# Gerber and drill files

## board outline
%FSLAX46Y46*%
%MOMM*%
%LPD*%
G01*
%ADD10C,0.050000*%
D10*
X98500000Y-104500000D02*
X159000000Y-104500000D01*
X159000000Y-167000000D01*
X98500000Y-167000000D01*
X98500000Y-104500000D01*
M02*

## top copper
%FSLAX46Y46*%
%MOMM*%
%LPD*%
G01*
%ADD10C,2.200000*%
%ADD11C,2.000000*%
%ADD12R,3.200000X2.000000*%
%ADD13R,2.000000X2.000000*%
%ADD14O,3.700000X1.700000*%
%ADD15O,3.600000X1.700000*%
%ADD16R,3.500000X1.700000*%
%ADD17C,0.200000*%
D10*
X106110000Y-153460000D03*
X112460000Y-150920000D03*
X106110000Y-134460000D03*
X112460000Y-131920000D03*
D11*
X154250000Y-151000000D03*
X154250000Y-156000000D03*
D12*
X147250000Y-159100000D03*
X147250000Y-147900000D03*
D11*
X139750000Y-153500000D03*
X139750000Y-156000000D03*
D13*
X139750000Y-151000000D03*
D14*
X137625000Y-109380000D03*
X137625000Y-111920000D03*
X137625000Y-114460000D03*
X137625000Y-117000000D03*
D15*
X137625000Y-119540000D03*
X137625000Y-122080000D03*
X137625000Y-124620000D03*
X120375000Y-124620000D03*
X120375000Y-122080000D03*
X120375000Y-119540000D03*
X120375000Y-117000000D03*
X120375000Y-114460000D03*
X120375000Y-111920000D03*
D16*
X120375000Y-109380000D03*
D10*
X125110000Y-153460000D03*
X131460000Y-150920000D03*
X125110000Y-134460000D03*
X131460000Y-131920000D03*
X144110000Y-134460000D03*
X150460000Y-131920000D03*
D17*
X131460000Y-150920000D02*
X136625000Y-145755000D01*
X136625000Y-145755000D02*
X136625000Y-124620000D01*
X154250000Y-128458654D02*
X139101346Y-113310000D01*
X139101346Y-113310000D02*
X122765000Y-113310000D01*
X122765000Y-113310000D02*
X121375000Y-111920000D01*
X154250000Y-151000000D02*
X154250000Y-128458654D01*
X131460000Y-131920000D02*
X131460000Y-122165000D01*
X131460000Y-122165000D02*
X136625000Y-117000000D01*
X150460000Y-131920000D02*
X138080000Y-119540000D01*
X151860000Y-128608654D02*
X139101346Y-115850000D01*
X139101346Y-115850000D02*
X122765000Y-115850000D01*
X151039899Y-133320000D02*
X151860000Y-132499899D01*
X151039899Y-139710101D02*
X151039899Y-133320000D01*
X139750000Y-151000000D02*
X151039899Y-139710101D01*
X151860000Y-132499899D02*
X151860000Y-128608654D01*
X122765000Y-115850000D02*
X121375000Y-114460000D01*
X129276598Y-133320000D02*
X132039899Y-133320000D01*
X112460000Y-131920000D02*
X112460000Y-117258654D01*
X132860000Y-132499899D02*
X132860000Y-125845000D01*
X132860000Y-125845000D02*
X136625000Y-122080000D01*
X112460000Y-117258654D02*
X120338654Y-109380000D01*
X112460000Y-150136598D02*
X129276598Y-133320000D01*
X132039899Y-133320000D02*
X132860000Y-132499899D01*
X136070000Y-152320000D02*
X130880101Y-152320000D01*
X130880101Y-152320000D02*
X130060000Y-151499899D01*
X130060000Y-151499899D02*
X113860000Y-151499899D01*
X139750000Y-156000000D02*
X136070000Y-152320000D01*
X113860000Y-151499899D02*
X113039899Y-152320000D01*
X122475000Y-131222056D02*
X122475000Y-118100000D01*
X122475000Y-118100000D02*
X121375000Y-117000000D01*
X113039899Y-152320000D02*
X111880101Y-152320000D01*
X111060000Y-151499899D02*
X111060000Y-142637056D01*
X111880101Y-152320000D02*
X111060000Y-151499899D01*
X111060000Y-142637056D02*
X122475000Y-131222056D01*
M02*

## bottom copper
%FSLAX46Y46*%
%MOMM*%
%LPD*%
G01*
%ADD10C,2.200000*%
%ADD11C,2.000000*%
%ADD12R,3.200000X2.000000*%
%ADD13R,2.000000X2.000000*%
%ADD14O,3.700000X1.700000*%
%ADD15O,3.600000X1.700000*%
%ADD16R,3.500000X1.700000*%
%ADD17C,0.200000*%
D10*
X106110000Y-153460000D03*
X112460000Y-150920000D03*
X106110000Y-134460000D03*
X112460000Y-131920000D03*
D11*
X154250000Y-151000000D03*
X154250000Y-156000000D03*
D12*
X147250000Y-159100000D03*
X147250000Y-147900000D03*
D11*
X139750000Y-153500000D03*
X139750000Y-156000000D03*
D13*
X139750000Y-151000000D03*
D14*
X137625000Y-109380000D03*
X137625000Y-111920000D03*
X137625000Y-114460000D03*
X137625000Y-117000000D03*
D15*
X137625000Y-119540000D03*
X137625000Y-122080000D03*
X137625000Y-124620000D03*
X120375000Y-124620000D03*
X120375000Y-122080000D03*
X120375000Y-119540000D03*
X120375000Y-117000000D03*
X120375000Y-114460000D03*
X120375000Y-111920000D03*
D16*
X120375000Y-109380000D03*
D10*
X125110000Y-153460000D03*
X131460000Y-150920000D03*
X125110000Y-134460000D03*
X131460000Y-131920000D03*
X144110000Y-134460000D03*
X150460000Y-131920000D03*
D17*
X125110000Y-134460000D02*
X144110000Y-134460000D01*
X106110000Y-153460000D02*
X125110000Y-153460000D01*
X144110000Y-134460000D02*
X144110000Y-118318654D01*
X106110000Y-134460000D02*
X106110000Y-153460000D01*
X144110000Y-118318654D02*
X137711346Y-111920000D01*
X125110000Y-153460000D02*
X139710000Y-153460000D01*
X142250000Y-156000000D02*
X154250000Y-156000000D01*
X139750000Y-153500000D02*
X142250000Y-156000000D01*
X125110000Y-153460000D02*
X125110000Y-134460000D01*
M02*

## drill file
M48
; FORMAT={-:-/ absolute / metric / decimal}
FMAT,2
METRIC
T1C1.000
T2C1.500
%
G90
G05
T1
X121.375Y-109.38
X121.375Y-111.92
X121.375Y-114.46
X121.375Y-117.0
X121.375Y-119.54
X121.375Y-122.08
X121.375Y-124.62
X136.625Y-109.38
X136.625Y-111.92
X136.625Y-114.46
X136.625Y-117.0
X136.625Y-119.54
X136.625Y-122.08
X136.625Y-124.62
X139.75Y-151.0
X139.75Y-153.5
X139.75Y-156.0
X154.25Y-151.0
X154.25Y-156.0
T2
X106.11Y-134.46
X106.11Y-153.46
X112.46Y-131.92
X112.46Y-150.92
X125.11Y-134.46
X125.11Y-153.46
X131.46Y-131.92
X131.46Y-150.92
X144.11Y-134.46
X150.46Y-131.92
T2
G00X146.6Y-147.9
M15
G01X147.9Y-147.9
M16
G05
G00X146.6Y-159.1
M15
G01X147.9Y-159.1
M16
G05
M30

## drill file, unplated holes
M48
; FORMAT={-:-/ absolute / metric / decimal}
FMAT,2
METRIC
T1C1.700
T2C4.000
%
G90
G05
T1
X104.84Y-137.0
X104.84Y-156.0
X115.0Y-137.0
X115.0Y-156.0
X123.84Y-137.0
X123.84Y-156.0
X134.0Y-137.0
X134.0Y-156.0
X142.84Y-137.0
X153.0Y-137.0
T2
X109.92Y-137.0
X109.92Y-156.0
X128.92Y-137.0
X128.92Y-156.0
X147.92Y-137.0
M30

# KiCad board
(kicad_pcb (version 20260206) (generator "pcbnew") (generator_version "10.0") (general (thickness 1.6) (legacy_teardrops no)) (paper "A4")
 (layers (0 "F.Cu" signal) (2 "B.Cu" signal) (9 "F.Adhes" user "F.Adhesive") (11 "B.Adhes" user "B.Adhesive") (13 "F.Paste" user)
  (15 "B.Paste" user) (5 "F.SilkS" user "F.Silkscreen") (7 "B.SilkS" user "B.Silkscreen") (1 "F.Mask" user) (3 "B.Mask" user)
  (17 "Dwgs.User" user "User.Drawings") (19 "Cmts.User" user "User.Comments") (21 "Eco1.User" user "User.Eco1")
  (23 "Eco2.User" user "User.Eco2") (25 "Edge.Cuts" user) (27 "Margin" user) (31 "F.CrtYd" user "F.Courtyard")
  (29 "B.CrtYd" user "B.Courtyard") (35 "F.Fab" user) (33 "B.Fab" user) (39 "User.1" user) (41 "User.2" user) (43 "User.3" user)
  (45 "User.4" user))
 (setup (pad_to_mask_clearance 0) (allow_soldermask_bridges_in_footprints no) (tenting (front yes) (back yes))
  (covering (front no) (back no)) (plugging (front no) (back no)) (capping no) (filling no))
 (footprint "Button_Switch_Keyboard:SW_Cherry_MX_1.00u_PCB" (layer "F.Cu") (at 112.46 150.92)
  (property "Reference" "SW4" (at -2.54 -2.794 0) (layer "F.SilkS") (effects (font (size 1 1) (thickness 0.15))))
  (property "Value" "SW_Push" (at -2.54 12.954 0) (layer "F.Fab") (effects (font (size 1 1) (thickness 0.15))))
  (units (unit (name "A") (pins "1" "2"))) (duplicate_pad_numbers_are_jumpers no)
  (pad "" np_thru_hole circle (at -7.62 5.08) (size 1.7 1.7) (drill 1.7) (layers "*.Cu" "*.Mask"))
  (pad "" np_thru_hole circle (at -2.54 5.08) (size 4 4) (drill 4) (layers "*.Cu" "*.Mask"))
  (pad "" np_thru_hole circle (at 2.54 5.08) (size 1.7 1.7) (drill 1.7) (layers "*.Cu" "*.Mask"))
  (pad "1" thru_hole circle (at 0 0) (size 2.2 2.2) (drill 1.5) (layers "*.Cu" "*.Mask") (remove_unused_layers no)
   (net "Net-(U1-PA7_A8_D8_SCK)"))
  (pad "2" thru_hole circle (at -6.35 2.54) (size 2.2 2.2) (drill 1.5) (layers "*.Cu" "*.Mask") (remove_unused_layers no)
   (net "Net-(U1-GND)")))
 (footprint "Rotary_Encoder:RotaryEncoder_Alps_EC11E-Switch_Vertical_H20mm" (layer "F.Cu") (at 139.75 151)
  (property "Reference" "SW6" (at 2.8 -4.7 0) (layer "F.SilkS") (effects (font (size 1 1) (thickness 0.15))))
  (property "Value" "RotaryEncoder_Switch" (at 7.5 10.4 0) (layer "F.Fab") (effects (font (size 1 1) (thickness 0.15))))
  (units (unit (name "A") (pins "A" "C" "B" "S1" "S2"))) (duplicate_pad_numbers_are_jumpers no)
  (pad "A" thru_hole rect (at 0 0) (size 2 2) (drill 1) (layers "*.Cu" "*.Mask") (remove_unused_layers no) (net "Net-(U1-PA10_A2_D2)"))
  (pad "B" thru_hole circle (at 0 5) (size 2 2) (drill 1) (layers "*.Cu" "*.Mask") (remove_unused_layers no) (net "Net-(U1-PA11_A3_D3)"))
  (pad "C" thru_hole circle (at 0 2.5) (size 2 2) (drill 1) (layers "*.Cu" "*.Mask") (remove_unused_layers no) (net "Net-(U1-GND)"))
  (pad "MP" thru_hole rect (at 7.5 -3.1) (size 3.2 2) (drill oval 2.8 1.5) (layers "*.Cu" "*.Mask") (remove_unused_layers no))
  (pad "MP" thru_hole rect (at 7.5 8.1) (size 3.2 2) (drill oval 2.8 1.5) (layers "*.Cu" "*.Mask") (remove_unused_layers no))
  (pad "S1" thru_hole circle (at 14.5 5) (size 2 2) (drill 1) (layers "*.Cu" "*.Mask") (remove_unused_layers no) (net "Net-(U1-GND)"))
  (pad "S2" thru_hole circle (at 14.5 0) (size 2 2) (drill 1) (layers "*.Cu" "*.Mask") (remove_unused_layers no) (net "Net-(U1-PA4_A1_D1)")))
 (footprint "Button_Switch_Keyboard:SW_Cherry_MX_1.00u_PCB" (layer "F.Cu") (at 131.46 150.92)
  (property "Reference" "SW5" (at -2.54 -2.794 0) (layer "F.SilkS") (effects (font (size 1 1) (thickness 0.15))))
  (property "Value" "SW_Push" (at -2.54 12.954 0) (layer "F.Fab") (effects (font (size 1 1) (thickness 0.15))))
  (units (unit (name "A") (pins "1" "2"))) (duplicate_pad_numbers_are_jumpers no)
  (pad "" np_thru_hole circle (at -7.62 5.08) (size 1.7 1.7) (drill 1.7) (layers "*.Cu" "*.Mask"))
  (pad "" np_thru_hole circle (at -2.54 5.08) (size 4 4) (drill 4) (layers "*.Cu" "*.Mask"))
  (pad "" np_thru_hole circle (at 2.54 5.08) (size 1.7 1.7) (drill 1.7) (layers "*.Cu" "*.Mask"))
  (pad "1" thru_hole circle (at 0 0) (size 2.2 2.2) (drill 1.5) (layers "*.Cu" "*.Mask") (remove_unused_layers no)
   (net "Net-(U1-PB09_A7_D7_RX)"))
  (pad "2" thru_hole circle (at -6.35 2.54) (size 2.2 2.2) (drill 1.5) (layers "*.Cu" "*.Mask") (remove_unused_layers no)
   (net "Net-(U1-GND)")))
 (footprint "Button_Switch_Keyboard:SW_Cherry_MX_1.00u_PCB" (layer "F.Cu") (at 150.46 131.92)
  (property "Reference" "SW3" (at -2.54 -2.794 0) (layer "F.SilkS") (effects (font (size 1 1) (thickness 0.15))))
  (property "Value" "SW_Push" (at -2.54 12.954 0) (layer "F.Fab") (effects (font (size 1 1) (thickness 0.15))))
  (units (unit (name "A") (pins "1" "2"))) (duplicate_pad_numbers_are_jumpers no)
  (pad "" np_thru_hole circle (at -7.62 5.08) (size 1.7 1.7) (drill 1.7) (layers "*.Cu" "*.Mask"))
  (pad "" np_thru_hole circle (at -2.54 5.08) (size 4 4) (drill 4) (layers "*.Cu" "*.Mask"))
  (pad "" np_thru_hole circle (at 2.54 5.08) (size 1.7 1.7) (drill 1.7) (layers "*.Cu" "*.Mask"))
  (pad "1" thru_hole circle (at 0 0) (size 2.2 2.2) (drill 1.5) (layers "*.Cu" "*.Mask") (remove_unused_layers no)
   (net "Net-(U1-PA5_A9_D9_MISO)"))
  (pad "2" thru_hole circle (at -6.35 2.54) (size 2.2 2.2) (drill 1.5) (layers "*.Cu" "*.Mask") (remove_unused_layers no)
   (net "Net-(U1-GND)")))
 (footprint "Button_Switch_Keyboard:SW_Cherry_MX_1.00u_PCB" (layer "F.Cu") (at 131.46 131.92)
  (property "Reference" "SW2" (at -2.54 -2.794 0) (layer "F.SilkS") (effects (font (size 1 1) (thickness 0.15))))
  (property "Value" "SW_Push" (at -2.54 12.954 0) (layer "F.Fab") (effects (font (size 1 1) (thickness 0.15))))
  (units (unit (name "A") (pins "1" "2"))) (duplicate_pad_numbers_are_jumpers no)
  (pad "" np_thru_hole circle (at -7.62 5.08) (size 1.7 1.7) (drill 1.7) (layers "*.Cu" "*.Mask"))
  (pad "" np_thru_hole circle (at -2.54 5.08) (size 4 4) (drill 4) (layers "*.Cu" "*.Mask"))
  (pad "" np_thru_hole circle (at 2.54 5.08) (size 1.7 1.7) (drill 1.7) (layers "*.Cu" "*.Mask"))
  (pad "1" thru_hole circle (at 0 0) (size 2.2 2.2) (drill 1.5) (layers "*.Cu" "*.Mask") (remove_unused_layers no)
   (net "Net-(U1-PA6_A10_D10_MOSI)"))
  (pad "2" thru_hole circle (at -6.35 2.54) (size 2.2 2.2) (drill 1.5) (layers "*.Cu" "*.Mask") (remove_unused_layers no)
   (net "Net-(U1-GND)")))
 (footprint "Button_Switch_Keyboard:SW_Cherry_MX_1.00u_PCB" (layer "F.Cu") (at 112.46 131.92)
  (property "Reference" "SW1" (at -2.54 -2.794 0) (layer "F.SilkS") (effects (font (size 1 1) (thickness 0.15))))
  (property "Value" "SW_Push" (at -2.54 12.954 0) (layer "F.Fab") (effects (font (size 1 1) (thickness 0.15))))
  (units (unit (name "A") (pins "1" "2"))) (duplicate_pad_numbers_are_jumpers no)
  (pad "" np_thru_hole circle (at -7.62 5.08) (size 1.7 1.7) (drill 1.7) (layers "*.Cu" "*.Mask"))
  (pad "" np_thru_hole circle (at -2.54 5.08) (size 4 4) (drill 4) (layers "*.Cu" "*.Mask"))
  (pad "" np_thru_hole circle (at 2.54 5.08) (size 1.7 1.7) (drill 1.7) (layers "*.Cu" "*.Mask"))
  (pad "1" thru_hole circle (at 0 0) (size 2.2 2.2) (drill 1.5) (layers "*.Cu" "*.Mask") (remove_unused_layers no)
   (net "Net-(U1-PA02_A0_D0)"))
  (pad "2" thru_hole circle (at -6.35 2.54) (size 2.2 2.2) (drill 1.5) (layers "*.Cu" "*.Mask") (remove_unused_layers no)
   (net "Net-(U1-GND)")))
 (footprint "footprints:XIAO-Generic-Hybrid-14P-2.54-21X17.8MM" (layer "F.Cu") (at 129 117)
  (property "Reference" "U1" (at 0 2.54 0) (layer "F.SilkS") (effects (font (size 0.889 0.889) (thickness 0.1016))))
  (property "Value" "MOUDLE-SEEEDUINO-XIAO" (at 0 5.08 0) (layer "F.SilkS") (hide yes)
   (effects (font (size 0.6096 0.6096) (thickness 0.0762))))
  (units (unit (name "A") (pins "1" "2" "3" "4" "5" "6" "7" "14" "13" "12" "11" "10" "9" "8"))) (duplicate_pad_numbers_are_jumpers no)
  (pad "1" thru_hole rect (at -7.625 -7.62) (size 3.5 1.7) (drill 1 (offset -1 0)) (layers "*.Cu" "*.Mask") (remove_unused_layers no)
   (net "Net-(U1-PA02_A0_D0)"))
  (pad "2" thru_hole oval (at -7.625 -5.08) (size 3.6 1.7) (drill 1 (offset -1 0)) (layers "*.Cu" "*.Mask") (remove_unused_layers no)
   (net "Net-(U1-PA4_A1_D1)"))
  (pad "3" thru_hole oval (at -7.625 -2.54) (size 3.6 1.7) (drill 1 (offset -1 0)) (layers "*.Cu" "*.Mask") (remove_unused_layers no)
   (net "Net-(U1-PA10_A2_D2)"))
  (pad "4" thru_hole oval (at -7.625 0) (size 3.6 1.7) (drill 1 (offset -1 0)) (layers "*.Cu" "*.Mask") (remove_unused_layers no)
   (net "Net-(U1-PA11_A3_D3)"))
  (pad "5" thru_hole oval (at -7.625 2.54) (size 3.6 1.7) (drill 1 (offset -1 0)) (layers "*.Cu" "*.Mask") (remove_unused_layers no)
   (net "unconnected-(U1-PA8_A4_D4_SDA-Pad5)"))
  (pad "6" thru_hole oval (at -7.625 5.08 180) (size 3.6 1.7) (drill 1 (offset 1 0)) (layers "*.Cu" "*.Mask") (remove_unused_layers no)
   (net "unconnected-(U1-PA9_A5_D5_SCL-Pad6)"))
  (pad "7" thru_hole oval (at -7.625 7.62) (size 3.6 1.7) (drill 1 (offset -1 0)) (layers "*.Cu" "*.Mask") (remove_unused_layers no)
   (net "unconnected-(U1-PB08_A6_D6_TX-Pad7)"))
  (pad "8" thru_hole oval (at 7.625 7.62) (size 3.6 1.7) (drill 1 (offset 1 0)) (layers "*.Cu" "*.Mask") (remove_unused_layers no)
   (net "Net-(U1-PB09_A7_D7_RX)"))
  (pad "9" thru_hole oval (at 7.625 5.08) (size 3.6 1.7) (drill 1 (offset 1 0)) (layers "*.Cu" "*.Mask") (remove_unused_layers no)
   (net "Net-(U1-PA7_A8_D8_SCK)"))
  (pad "10" thru_hole oval (at 7.625 2.54) (size 3.6 1.7) (drill 1 (offset 1 0)) (layers "*.Cu" "*.Mask") (remove_unused_layers no)
   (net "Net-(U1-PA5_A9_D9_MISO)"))
  (pad "11" thru_hole oval (at 7.625 0) (size 3.7 1.7) (drill 1 (offset 1 0)) (layers "*.Cu" "*.Mask") (remove_unused_layers no)
   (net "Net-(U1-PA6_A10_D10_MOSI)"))
  (pad "12" thru_hole oval (at 7.625 -2.54) (size 3.7 1.7) (drill 1 (offset 1 0)) (layers "*.Cu" "*.Mask") (remove_unused_layers no)
   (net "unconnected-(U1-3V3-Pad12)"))
  (pad "13" thru_hole oval (at 7.625 -5.08) (size 3.7 1.7) (drill 1 (offset 1 0)) (layers "*.Cu" "*.Mask") (remove_unused_layers no)
   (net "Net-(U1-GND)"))
  (pad "14" thru_hole oval (at 7.625 -7.62) (size 3.7 1.7) (drill 1 (offset 1 0)) (layers "*.Cu" "*.Mask") (remove_unused_layers no)
   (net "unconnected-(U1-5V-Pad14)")))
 (gr_rect (start 98.5 104.5) (end 159 167) (stroke (width 0.05) (type default)) (fill no) (layer "Edge.Cuts"))
 (segment (start 112.46 131.92) (end 112.46 117.258654) (width 0.2) (layer "F.Cu") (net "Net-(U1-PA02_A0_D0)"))
 (segment (start 112.46 117.258654) (end 120.338654 109.38) (width 0.2) (layer "F.Cu") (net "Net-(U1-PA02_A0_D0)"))
 (segment (start 131.46 131.92) (end 131.46 122.165) (width 0.2) (layer "F.Cu") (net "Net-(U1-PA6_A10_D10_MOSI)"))
 (segment (start 131.46 122.165) (end 136.625 117) (width 0.2) (layer "F.Cu") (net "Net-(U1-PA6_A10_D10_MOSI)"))
 (segment (start 150.46 131.92) (end 138.08 119.54) (width 0.2) (layer "F.Cu") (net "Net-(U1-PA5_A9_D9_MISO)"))
 (segment (start 112.46 150.136598) (end 129.276598 133.32) (width 0.2) (layer "F.Cu") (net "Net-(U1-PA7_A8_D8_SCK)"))
 (segment (start 132.86 132.499899) (end 132.86 125.845) (width 0.2) (layer "F.Cu") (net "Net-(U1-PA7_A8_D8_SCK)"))
 (segment (start 129.276598 133.32) (end 132.039899 133.32) (width 0.2) (layer "F.Cu") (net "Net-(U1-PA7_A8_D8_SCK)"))
 (segment (start 132.86 125.845) (end 136.625 122.08) (width 0.2) (layer "F.Cu") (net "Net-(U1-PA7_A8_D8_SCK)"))
 (segment (start 132.039899 133.32) (end 132.86 132.499899) (width 0.2) (layer "F.Cu") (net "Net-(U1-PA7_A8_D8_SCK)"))
 (segment (start 131.46 150.92) (end 136.625 145.755) (width 0.2) (layer "F.Cu") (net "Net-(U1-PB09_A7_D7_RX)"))
 (segment (start 136.625 145.755) (end 136.625 124.62) (width 0.2) (layer "F.Cu") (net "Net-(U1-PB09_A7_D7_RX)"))
 (segment (start 130.06 151.499899) (end 113.86 151.499899) (width 0.2) (layer "F.Cu") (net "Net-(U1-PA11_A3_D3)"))
 (segment (start 122.475 131.222056) (end 122.475 118.1) (width 0.2) (layer "F.Cu") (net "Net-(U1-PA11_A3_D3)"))
 (segment (start 111.06 142.637056) (end 122.475 131.222056) (width 0.2) (layer "F.Cu") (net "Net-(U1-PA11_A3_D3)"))
 (segment (start 111.880101 152.32) (end 111.06 151.499899) (width 0.2) (layer "F.Cu") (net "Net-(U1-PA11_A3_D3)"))
 (segment (start 136.07 152.32) (end 130.880101 152.32) (width 0.2) (layer "F.Cu") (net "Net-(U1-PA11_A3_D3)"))
 (segment (start 111.06 151.499899) (end 111.06 142.637056) (width 0.2) (layer "F.Cu") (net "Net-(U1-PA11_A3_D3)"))
 (segment (start 130.880101 152.32) (end 130.06 151.499899) (width 0.2) (layer "F.Cu") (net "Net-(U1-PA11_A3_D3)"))
 (segment (start 113.039899 152.32) (end 111.880101 152.32) (width 0.2) (layer "F.Cu") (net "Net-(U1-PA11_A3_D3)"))
 (segment (start 139.75 156) (end 136.07 152.32) (width 0.2) (layer "F.Cu") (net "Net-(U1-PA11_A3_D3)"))
 (segment (start 122.475 118.1) (end 121.375 117) (width 0.2) (layer "F.Cu") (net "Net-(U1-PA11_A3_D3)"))
 (segment (start 113.86 151.499899) (end 113.039899 152.32) (width 0.2) (layer "F.Cu") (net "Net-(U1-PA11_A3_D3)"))
 (segment (start 151.039899 133.32) (end 151.86 132.499899) (width 0.2) (layer "F.Cu") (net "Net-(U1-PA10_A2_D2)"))
 (segment (start 139.75 151) (end 151.039899 139.710101) (width 0.2) (layer "F.Cu") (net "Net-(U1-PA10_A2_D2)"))
 (segment (start 139.101346 115.85) (end 122.765 115.85) (width 0.2) (layer "F.Cu") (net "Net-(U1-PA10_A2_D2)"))
 (segment (start 122.765 115.85) (end 121.375 114.46) (width 0.2) (layer "F.Cu") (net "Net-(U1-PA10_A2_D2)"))
 (segment (start 151.86 132.499899) (end 151.86 128.608654) (width 0.2) (layer "F.Cu") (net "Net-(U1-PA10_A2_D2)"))
 (segment (start 151.86 128.608654) (end 139.101346 115.85) (width 0.2) (layer "F.Cu") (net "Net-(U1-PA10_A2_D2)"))
 (segment (start 151.039899 139.710101) (end 151.039899 133.32) (width 0.2) (layer "F.Cu") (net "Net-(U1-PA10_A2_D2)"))
 (segment (start 154.25 151) (end 154.25 128.458654) (width 0.2) (layer "F.Cu") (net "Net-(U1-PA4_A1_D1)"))
 (segment (start 154.25 128.458654) (end 139.101346 113.31) (width 0.2) (layer "F.Cu") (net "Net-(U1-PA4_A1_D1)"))
 (segment (start 139.101346 113.31) (end 122.765 113.31) (width 0.2) (layer "F.Cu") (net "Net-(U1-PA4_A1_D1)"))
 (segment (start 122.765 113.31) (end 121.375 111.92) (width 0.2) (layer "F.Cu") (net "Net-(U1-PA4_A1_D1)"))
 (segment (start 125.11 134.46) (end 144.11 134.46) (width 0.2) (layer "B.Cu") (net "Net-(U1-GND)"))
 (segment (start 142.25 156) (end 154.25 156) (width 0.2) (layer "B.Cu") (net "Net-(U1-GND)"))
 (segment (start 106.11 134.46) (end 106.11 153.46) (width 0.2) (layer "B.Cu") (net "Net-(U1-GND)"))
 (segment (start 106.11 153.46) (end 125.11 153.46) (width 0.2) (layer "B.Cu") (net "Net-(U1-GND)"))
 (segment (start 144.11 118.318654) (end 137.711346 111.92) (width 0.2) (layer "B.Cu") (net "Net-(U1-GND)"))
 (segment (start 125.11 153.46) (end 139.71 153.46) (width 0.2) (layer "B.Cu") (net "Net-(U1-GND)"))
 (segment (start 144.11 134.46) (end 144.11 118.318654) (width 0.2) (layer "B.Cu") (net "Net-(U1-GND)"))
 (segment (start 139.75 153.5) (end 142.25 156) (width 0.2) (layer "B.Cu") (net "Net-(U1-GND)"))
 (segment (start 125.11 153.46) (end 125.11 134.46) (width 0.2) (layer "B.Cu") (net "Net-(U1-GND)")))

